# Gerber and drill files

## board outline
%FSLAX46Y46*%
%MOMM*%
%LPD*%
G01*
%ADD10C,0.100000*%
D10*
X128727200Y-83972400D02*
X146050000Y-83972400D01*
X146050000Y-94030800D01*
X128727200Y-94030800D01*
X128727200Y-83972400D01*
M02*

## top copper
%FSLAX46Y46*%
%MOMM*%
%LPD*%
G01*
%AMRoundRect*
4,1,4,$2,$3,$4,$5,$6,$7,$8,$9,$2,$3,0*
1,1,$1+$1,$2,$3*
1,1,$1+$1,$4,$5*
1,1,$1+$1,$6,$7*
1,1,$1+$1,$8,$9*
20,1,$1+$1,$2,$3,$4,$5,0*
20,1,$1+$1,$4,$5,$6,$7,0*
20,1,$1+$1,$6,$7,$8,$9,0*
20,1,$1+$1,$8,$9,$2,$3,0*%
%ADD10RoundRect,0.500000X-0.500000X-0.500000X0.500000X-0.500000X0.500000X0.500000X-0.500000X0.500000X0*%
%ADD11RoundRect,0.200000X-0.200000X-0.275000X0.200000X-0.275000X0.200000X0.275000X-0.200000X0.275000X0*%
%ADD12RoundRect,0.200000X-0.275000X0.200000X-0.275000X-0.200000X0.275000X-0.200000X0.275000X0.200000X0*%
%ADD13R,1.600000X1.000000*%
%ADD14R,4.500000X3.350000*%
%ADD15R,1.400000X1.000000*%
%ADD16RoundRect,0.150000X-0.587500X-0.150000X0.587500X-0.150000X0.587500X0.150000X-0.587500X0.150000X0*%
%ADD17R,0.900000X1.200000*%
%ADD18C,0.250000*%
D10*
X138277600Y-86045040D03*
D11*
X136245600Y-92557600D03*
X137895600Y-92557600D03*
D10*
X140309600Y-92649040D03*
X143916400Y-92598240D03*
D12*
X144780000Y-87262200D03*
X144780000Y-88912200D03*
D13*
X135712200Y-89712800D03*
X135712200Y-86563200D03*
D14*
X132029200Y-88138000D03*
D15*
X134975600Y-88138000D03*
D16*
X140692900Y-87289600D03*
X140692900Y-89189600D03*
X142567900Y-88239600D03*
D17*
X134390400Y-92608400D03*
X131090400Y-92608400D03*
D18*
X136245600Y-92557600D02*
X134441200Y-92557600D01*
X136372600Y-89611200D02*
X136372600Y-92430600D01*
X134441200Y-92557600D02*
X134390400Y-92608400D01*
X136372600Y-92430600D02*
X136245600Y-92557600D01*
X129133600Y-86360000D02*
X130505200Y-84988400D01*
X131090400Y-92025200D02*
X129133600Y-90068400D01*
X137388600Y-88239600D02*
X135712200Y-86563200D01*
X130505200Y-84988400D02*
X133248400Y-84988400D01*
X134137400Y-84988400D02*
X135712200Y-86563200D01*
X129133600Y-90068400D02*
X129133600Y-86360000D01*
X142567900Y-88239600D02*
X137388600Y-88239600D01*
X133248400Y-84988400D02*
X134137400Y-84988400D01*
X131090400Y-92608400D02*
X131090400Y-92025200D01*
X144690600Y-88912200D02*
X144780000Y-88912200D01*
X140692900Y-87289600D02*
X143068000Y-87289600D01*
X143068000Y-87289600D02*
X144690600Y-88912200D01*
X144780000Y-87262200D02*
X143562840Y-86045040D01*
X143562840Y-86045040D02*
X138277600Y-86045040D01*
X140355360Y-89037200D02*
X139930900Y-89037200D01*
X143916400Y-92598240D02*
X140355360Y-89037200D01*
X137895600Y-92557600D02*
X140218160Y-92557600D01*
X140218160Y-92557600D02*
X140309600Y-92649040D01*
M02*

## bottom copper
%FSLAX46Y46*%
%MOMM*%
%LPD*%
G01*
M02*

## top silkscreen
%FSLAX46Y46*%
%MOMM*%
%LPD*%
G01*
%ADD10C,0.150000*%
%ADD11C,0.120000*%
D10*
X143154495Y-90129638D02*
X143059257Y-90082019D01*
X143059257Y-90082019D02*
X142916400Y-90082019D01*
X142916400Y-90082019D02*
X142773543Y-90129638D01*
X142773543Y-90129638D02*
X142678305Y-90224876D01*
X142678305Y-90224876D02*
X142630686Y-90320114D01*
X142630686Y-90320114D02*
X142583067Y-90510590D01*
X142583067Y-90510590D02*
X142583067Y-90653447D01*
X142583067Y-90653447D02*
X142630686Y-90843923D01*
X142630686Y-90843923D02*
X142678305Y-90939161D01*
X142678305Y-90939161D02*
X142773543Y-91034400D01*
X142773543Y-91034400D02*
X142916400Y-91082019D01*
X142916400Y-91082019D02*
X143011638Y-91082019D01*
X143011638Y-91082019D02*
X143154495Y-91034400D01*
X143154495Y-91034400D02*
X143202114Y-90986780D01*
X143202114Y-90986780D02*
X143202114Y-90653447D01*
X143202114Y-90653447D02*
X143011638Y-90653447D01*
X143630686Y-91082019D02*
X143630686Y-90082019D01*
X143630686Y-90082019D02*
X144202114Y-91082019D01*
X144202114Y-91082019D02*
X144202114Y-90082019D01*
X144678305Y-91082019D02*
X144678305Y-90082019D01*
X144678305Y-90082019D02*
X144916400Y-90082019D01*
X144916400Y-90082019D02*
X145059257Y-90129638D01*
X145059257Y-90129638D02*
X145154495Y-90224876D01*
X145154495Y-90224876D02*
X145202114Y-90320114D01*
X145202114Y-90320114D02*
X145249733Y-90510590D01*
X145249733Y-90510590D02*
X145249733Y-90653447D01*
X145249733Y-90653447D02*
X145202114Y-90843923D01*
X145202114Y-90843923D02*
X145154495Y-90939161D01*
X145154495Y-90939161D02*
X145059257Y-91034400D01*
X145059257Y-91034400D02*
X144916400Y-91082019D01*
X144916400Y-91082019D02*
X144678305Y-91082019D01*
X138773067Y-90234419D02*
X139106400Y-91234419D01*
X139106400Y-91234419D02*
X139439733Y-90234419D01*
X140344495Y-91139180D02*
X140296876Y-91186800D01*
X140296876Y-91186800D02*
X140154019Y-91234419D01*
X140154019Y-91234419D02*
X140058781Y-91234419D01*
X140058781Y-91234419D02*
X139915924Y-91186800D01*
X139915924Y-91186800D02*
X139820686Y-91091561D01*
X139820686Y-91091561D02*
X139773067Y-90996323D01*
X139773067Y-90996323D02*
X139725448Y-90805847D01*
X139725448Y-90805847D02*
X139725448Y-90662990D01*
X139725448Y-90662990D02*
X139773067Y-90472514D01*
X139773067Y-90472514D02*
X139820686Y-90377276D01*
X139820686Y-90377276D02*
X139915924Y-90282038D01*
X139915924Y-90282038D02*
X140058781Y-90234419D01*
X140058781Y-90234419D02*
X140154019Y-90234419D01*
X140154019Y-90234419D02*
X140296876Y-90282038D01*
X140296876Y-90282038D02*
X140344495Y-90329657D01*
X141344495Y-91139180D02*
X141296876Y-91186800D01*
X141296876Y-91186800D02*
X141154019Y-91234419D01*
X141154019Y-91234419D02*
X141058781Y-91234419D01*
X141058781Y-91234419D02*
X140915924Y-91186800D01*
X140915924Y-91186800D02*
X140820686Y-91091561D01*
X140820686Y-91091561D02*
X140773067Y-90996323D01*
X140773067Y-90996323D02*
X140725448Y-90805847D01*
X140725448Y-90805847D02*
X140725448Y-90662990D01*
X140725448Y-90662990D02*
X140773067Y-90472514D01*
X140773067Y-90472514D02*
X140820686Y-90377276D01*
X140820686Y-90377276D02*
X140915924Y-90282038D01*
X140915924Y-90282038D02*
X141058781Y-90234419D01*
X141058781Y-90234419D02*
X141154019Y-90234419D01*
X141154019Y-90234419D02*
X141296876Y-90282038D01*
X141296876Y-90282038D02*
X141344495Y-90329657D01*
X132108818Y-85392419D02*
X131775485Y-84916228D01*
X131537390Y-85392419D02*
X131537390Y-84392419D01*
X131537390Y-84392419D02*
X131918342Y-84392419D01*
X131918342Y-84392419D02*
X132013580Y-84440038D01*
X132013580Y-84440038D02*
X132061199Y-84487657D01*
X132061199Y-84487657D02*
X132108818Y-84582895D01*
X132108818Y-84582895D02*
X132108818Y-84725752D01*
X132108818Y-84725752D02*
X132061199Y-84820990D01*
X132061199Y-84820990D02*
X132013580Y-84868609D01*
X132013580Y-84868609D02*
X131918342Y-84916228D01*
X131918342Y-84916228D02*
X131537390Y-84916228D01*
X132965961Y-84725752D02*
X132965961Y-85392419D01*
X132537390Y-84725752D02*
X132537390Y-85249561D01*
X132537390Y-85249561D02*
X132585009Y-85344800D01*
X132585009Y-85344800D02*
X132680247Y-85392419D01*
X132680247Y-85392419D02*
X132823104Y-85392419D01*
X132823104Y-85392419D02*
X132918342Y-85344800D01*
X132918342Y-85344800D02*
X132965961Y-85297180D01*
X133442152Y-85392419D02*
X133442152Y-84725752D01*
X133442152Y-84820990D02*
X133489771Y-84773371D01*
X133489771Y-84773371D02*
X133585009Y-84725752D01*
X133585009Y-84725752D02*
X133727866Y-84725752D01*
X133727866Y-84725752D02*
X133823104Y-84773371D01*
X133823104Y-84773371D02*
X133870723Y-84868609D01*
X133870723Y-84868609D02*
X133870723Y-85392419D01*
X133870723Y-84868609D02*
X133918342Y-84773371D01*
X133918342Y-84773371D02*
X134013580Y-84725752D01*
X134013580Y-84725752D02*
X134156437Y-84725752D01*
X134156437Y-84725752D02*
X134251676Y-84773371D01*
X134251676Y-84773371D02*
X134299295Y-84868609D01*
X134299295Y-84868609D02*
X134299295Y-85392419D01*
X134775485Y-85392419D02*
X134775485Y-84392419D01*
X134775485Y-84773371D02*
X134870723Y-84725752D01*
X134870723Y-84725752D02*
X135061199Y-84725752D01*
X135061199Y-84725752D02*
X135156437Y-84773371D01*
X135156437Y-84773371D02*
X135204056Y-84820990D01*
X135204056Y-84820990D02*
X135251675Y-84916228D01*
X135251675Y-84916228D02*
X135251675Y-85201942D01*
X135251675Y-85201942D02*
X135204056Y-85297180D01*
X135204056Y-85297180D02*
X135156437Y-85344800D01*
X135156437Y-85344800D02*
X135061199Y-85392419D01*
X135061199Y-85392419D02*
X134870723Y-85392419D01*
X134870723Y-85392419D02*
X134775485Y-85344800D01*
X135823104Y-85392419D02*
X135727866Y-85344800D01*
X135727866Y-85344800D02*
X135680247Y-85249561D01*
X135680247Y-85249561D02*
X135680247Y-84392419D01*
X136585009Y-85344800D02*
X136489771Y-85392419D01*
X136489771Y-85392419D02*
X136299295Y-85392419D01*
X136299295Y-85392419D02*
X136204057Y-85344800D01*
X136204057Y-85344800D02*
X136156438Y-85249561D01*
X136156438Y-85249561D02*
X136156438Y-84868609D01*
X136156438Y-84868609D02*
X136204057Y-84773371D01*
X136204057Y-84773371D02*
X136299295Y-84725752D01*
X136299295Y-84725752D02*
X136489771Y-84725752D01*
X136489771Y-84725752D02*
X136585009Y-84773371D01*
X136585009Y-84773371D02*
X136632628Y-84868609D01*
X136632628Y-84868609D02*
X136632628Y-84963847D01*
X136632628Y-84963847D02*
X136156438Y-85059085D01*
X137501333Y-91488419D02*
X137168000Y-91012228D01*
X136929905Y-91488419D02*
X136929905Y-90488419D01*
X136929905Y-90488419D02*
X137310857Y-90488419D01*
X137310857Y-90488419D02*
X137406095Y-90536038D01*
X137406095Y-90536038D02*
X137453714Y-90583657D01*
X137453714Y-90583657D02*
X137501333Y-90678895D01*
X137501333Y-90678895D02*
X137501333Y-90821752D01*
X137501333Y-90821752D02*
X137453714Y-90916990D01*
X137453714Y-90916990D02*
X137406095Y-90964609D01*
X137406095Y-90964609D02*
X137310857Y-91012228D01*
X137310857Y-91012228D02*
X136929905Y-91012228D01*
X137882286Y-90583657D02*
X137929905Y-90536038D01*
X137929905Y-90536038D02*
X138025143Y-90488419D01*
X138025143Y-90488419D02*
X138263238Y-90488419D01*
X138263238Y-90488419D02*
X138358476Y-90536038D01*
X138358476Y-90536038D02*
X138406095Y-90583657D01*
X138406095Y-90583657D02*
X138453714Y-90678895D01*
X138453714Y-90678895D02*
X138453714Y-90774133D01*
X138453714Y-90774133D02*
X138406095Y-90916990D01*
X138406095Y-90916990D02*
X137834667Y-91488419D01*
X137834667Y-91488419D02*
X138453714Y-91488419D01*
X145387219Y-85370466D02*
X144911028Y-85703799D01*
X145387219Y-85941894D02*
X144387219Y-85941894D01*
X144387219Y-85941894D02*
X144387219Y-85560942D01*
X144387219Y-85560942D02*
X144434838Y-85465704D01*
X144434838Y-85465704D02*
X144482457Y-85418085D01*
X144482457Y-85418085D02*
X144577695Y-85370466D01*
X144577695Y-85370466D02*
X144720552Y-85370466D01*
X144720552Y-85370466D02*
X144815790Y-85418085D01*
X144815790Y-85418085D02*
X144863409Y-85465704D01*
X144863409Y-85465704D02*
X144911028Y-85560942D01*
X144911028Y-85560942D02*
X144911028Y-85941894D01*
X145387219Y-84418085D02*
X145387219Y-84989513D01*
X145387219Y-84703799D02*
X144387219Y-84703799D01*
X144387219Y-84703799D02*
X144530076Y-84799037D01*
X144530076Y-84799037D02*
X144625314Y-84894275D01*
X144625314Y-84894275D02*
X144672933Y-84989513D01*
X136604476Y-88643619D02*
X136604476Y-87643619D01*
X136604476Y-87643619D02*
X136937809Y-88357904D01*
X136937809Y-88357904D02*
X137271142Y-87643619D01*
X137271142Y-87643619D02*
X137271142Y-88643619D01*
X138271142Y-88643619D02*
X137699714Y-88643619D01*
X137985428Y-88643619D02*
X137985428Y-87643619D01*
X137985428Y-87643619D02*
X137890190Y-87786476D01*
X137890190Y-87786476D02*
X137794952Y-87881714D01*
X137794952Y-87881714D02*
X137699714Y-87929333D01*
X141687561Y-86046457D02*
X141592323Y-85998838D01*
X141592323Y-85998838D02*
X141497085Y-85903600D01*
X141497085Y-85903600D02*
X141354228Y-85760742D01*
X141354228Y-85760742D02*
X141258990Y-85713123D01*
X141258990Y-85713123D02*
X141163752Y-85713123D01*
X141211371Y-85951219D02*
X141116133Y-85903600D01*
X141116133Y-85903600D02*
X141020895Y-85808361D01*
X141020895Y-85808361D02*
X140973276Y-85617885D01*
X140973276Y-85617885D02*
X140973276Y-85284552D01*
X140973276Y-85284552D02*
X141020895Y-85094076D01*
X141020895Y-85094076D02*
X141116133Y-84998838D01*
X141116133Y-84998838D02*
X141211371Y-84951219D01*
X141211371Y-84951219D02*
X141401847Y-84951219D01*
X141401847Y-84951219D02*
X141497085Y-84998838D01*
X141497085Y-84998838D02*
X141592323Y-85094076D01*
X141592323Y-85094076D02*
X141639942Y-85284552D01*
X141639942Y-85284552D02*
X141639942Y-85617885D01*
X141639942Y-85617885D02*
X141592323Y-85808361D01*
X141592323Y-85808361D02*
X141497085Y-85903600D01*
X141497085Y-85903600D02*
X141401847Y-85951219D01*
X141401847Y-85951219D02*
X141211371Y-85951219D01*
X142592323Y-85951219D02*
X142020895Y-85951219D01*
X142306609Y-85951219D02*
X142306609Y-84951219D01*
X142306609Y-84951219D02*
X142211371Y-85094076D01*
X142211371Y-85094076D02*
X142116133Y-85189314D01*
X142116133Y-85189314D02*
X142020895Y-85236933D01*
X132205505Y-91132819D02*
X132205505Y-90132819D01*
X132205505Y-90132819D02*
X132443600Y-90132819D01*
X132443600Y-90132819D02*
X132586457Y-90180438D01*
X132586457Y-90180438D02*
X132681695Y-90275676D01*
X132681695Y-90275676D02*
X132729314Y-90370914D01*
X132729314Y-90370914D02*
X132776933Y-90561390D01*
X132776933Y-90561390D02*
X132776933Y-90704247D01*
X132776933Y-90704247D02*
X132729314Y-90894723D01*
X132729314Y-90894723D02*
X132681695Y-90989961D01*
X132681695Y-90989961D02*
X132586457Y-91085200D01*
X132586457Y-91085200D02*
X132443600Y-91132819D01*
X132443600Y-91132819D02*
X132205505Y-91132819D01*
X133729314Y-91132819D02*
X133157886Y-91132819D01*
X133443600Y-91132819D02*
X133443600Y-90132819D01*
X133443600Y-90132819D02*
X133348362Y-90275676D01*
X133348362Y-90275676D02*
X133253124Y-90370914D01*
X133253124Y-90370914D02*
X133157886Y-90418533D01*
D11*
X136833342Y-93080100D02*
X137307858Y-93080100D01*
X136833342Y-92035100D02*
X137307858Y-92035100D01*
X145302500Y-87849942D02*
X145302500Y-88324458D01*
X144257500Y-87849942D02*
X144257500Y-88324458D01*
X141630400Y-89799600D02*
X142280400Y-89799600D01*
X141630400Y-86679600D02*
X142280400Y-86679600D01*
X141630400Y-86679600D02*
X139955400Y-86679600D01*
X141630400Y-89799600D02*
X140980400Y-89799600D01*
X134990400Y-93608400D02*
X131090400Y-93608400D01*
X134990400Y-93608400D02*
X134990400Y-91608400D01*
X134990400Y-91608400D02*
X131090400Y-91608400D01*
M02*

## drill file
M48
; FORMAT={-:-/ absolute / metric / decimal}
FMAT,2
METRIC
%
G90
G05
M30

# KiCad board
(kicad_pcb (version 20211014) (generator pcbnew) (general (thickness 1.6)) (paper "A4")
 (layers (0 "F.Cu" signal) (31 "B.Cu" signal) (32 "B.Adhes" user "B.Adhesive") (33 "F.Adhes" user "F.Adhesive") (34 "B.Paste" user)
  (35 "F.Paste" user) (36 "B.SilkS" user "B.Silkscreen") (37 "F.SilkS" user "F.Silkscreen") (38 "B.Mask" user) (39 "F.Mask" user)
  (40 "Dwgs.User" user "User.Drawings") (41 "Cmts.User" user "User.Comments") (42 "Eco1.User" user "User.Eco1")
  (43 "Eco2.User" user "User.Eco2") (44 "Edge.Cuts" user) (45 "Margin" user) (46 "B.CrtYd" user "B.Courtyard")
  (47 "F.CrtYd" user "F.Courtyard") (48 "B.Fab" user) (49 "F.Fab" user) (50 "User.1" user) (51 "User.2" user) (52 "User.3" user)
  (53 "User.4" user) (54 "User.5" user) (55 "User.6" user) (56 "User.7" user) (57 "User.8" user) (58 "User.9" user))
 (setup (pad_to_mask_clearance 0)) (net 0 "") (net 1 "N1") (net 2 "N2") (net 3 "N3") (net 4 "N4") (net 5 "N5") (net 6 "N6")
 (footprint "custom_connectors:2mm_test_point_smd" (layer "F.Cu") (at 138.2776 86.0552)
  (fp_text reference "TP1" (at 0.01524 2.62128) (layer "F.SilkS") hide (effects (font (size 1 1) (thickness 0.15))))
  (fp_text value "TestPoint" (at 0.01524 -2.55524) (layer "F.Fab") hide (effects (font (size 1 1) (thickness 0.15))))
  (pad "1" smd roundrect locked (at 0 -0.01016) (size 2 2) (layers "F.Cu" "F.Paste" "F.Mask") (roundrect_rratio 0.25) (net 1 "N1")))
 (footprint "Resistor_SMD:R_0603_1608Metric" (layer "F.Cu") (at 137.0706 92.5576)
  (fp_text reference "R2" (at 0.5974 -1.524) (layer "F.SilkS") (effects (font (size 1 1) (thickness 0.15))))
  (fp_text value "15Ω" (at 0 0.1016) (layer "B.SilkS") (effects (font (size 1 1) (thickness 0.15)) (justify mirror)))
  (fp_line (start -0.237258 0.5225) (end 0.237258 0.5225) (layer "F.SilkS") (width 0.12))
  (fp_line (start -0.237258 -0.5225) (end 0.237258 -0.5225) (layer "F.SilkS") (width 0.12))
  (pad "1" smd roundrect (at -0.825 0) (size 0.8 0.95) (layers "F.Cu" "F.Paste" "F.Mask") (roundrect_rratio 0.25) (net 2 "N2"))
  (pad "2" smd roundrect (at 0.825 0) (size 0.8 0.95) (layers "F.Cu" "F.Paste" "F.Mask") (roundrect_rratio 0.25) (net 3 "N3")))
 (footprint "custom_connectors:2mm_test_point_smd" (layer "F.Cu") (at 140.3096 92.6592)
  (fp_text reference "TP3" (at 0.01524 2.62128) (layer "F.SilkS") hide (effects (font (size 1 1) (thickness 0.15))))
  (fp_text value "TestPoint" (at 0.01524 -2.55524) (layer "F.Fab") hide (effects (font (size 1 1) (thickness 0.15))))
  (pad "1" smd roundrect locked (at 0 -0.01016) (size 2 2) (layers "F.Cu" "F.Paste" "F.Mask") (roundrect_rratio 0.25) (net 3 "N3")))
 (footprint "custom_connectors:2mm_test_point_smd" (layer "F.Cu") (at 143.9164 92.6084)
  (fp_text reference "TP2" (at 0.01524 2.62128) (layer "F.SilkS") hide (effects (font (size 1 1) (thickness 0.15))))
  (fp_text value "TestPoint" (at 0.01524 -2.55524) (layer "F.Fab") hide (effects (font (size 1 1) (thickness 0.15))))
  (pad "1" smd roundrect locked (at 0 -0.01016) (size 2 2) (layers "F.Cu" "F.Paste" "F.Mask") (roundrect_rratio 0.25) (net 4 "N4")))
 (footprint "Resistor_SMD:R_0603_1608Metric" (layer "F.Cu") (at 144.78 88.0872 -90)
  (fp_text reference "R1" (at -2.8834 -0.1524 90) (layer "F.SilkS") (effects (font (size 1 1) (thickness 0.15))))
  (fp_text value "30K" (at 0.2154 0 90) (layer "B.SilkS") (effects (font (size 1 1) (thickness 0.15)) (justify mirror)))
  (fp_line (start -0.237258 -0.5225) (end 0.237258 -0.5225) (layer "F.SilkS") (width 0.12))
  (fp_line (start -0.237258 0.5225) (end 0.237258 0.5225) (layer "F.SilkS") (width 0.12))
  (pad "1" smd roundrect (at -0.825 0 270) (size 0.8 0.95) (layers "F.Cu" "F.Paste" "F.Mask") (roundrect_rratio 0.25) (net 1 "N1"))
  (pad "2" smd roundrect (at 0.825 0 270) (size 0.8 0.95) (layers "F.Cu" "F.Paste" "F.Mask") (roundrect_rratio 0.25) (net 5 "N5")))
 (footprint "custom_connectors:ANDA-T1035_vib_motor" (layer "F.Cu") (at 134.9756 88.138)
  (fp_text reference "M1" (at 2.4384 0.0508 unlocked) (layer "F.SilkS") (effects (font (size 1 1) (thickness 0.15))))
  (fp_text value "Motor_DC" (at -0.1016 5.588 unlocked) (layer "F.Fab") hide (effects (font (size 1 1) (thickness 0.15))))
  (pad "1" smd rect (at 0.7366 1.5748) (size 1.6 1) (layers "F.Cu" "F.Paste" "F.Mask") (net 2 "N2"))
  (pad "2" smd rect (at 0.7366 -1.5748) (size 1.6 1) (layers "F.Cu" "F.Paste" "F.Mask") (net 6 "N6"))
  (pad "3" smd rect (at -2.9464 0) (size 4.5 3.35) (layers "F.Cu" "F.Paste" "F.Mask"))
  (pad "3" smd rect (at 0 0) (size 1.4 1) (layers "F.Cu" "F.Paste" "F.Mask")))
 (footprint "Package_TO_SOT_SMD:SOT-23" (layer "F.Cu") (at 141.6304 88.2396)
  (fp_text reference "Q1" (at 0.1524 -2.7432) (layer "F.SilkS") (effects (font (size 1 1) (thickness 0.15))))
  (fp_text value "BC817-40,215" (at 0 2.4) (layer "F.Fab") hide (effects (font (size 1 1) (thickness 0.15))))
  (fp_line (start 0 1.56) (end 0.65 1.56) (layer "F.SilkS") (width 0.12))
  (fp_line (start 0 -1.56) (end 0.65 -1.56) (layer "F.SilkS") (width 0.12))
  (fp_line (start 0 -1.56) (end -1.675 -1.56) (layer "F.SilkS") (width 0.12))
  (fp_line (start 0 1.56) (end -0.65 1.56) (layer "F.SilkS") (width 0.12))
  (pad "1" smd roundrect (at -0.9375 -0.95) (size 1.475 0.6) (layers "F.Cu" "F.Paste" "F.Mask") (roundrect_rratio 0.25) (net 5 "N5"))
  (pad "2" smd roundrect (at -0.9375 0.95) (size 1.475 0.6) (layers "F.Cu" "F.Paste" "F.Mask") (roundrect_rratio 0.25) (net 4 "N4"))
  (pad "3" smd roundrect (at 0.9375 0) (size 1.475 0.6) (layers "F.Cu" "F.Paste" "F.Mask") (roundrect_rratio 0.25) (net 6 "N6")))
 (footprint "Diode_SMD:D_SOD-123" (layer "F.Cu") (at 132.7404 92.6084 180)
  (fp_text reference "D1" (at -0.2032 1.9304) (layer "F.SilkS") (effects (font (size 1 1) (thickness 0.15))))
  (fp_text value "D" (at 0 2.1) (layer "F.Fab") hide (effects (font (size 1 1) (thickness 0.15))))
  (fp_line (start -2.25 -1) (end 1.65 -1) (layer "F.SilkS") (width 0.12))
  (fp_line (start -2.25 -1) (end -2.25 1) (layer "F.SilkS") (width 0.12))
  (fp_line (start -2.25 1) (end 1.65 1) (layer "F.SilkS") (width 0.12))
  (pad "1" smd rect (at -1.65 0 180) (size 0.9 1.2) (layers "F.Cu" "F.Paste" "F.Mask") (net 2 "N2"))
  (pad "2" smd rect (at 1.65 0 180) (size 0.9 1.2) (layers "F.Cu" "F.Paste" "F.Mask") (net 6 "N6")))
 (gr_rect (start 128.7272 83.9724) (end 146.05 94.0308) (layer "Edge.Cuts") (width 0.1) (fill none))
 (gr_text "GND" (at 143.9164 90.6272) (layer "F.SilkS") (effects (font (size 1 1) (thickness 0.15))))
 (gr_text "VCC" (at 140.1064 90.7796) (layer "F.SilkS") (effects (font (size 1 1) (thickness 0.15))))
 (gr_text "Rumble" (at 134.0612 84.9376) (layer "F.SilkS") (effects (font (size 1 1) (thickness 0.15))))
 (segment (start 136.2456 92.5576) (end 134.4412 92.5576) (width 0.25) (layer "F.Cu") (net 2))
 (segment (start 136.3726 89.6112) (end 136.3726 92.4306) (width 0.25) (layer "F.Cu") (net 2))
 (segment (start 134.4412 92.5576) (end 134.3904 92.6084) (width 0.25) (layer "F.Cu") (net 2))
 (segment (start 136.3726 92.4306) (end 136.2456 92.5576) (width 0.25) (layer "F.Cu") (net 2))
 (segment (start 129.1336 86.36) (end 130.5052 84.9884) (width 0.25) (layer "F.Cu") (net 6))
 (segment (start 131.0904 92.0252) (end 129.1336 90.0684) (width 0.25) (layer "F.Cu") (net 6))
 (segment (start 137.3886 88.2396) (end 135.7122 86.5632) (width 0.25) (layer "F.Cu") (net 6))
 (segment (start 130.5052 84.9884) (end 133.2484 84.9884) (width 0.25) (layer "F.Cu") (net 6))
 (segment (start 134.1374 84.9884) (end 135.7122 86.5632) (width 0.25) (layer "F.Cu") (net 6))
 (segment (start 129.1336 90.0684) (end 129.1336 86.36) (width 0.25) (layer "F.Cu") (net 6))
 (segment (start 142.5679 88.2396) (end 137.3886 88.2396) (width 0.25) (layer "F.Cu") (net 6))
 (segment (start 133.2484 84.9884) (end 134.1374 84.9884) (width 0.25) (layer "F.Cu") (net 6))
 (segment (start 131.0904 92.6084) (end 131.0904 92.0252) (width 0.25) (layer "F.Cu") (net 6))
 (segment (start 144.6906 88.9122) (end 144.78 88.9122) (width 0.25) (layer "F.Cu") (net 5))
 (segment (start 140.6929 87.2896) (end 143.068 87.2896) (width 0.25) (layer "F.Cu") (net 5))
 (segment (start 143.068 87.2896) (end 144.6906 88.9122) (width 0.25) (layer "F.Cu") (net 5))
 (segment (start 144.78 87.2622) (end 143.56284 86.04504) (width 0.25) (layer "F.Cu") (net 1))
 (segment (start 143.56284 86.04504) (end 138.2776 86.04504) (width 0.25) (layer "F.Cu") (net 1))
 (segment (start 140.35536 89.0372) (end 139.9309 89.0372) (width 0.25) (layer "F.Cu") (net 4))
 (segment (start 143.9164 92.59824) (end 140.35536 89.0372) (width 0.25) (layer "F.Cu") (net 4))
 (segment (start 137.8956 92.5576) (end 140.21816 92.5576) (width 0.25) (layer "F.Cu") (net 3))
 (segment (start 140.21816 92.5576) (end 140.3096 92.64904) (width 0.25) (layer "F.Cu") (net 3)))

